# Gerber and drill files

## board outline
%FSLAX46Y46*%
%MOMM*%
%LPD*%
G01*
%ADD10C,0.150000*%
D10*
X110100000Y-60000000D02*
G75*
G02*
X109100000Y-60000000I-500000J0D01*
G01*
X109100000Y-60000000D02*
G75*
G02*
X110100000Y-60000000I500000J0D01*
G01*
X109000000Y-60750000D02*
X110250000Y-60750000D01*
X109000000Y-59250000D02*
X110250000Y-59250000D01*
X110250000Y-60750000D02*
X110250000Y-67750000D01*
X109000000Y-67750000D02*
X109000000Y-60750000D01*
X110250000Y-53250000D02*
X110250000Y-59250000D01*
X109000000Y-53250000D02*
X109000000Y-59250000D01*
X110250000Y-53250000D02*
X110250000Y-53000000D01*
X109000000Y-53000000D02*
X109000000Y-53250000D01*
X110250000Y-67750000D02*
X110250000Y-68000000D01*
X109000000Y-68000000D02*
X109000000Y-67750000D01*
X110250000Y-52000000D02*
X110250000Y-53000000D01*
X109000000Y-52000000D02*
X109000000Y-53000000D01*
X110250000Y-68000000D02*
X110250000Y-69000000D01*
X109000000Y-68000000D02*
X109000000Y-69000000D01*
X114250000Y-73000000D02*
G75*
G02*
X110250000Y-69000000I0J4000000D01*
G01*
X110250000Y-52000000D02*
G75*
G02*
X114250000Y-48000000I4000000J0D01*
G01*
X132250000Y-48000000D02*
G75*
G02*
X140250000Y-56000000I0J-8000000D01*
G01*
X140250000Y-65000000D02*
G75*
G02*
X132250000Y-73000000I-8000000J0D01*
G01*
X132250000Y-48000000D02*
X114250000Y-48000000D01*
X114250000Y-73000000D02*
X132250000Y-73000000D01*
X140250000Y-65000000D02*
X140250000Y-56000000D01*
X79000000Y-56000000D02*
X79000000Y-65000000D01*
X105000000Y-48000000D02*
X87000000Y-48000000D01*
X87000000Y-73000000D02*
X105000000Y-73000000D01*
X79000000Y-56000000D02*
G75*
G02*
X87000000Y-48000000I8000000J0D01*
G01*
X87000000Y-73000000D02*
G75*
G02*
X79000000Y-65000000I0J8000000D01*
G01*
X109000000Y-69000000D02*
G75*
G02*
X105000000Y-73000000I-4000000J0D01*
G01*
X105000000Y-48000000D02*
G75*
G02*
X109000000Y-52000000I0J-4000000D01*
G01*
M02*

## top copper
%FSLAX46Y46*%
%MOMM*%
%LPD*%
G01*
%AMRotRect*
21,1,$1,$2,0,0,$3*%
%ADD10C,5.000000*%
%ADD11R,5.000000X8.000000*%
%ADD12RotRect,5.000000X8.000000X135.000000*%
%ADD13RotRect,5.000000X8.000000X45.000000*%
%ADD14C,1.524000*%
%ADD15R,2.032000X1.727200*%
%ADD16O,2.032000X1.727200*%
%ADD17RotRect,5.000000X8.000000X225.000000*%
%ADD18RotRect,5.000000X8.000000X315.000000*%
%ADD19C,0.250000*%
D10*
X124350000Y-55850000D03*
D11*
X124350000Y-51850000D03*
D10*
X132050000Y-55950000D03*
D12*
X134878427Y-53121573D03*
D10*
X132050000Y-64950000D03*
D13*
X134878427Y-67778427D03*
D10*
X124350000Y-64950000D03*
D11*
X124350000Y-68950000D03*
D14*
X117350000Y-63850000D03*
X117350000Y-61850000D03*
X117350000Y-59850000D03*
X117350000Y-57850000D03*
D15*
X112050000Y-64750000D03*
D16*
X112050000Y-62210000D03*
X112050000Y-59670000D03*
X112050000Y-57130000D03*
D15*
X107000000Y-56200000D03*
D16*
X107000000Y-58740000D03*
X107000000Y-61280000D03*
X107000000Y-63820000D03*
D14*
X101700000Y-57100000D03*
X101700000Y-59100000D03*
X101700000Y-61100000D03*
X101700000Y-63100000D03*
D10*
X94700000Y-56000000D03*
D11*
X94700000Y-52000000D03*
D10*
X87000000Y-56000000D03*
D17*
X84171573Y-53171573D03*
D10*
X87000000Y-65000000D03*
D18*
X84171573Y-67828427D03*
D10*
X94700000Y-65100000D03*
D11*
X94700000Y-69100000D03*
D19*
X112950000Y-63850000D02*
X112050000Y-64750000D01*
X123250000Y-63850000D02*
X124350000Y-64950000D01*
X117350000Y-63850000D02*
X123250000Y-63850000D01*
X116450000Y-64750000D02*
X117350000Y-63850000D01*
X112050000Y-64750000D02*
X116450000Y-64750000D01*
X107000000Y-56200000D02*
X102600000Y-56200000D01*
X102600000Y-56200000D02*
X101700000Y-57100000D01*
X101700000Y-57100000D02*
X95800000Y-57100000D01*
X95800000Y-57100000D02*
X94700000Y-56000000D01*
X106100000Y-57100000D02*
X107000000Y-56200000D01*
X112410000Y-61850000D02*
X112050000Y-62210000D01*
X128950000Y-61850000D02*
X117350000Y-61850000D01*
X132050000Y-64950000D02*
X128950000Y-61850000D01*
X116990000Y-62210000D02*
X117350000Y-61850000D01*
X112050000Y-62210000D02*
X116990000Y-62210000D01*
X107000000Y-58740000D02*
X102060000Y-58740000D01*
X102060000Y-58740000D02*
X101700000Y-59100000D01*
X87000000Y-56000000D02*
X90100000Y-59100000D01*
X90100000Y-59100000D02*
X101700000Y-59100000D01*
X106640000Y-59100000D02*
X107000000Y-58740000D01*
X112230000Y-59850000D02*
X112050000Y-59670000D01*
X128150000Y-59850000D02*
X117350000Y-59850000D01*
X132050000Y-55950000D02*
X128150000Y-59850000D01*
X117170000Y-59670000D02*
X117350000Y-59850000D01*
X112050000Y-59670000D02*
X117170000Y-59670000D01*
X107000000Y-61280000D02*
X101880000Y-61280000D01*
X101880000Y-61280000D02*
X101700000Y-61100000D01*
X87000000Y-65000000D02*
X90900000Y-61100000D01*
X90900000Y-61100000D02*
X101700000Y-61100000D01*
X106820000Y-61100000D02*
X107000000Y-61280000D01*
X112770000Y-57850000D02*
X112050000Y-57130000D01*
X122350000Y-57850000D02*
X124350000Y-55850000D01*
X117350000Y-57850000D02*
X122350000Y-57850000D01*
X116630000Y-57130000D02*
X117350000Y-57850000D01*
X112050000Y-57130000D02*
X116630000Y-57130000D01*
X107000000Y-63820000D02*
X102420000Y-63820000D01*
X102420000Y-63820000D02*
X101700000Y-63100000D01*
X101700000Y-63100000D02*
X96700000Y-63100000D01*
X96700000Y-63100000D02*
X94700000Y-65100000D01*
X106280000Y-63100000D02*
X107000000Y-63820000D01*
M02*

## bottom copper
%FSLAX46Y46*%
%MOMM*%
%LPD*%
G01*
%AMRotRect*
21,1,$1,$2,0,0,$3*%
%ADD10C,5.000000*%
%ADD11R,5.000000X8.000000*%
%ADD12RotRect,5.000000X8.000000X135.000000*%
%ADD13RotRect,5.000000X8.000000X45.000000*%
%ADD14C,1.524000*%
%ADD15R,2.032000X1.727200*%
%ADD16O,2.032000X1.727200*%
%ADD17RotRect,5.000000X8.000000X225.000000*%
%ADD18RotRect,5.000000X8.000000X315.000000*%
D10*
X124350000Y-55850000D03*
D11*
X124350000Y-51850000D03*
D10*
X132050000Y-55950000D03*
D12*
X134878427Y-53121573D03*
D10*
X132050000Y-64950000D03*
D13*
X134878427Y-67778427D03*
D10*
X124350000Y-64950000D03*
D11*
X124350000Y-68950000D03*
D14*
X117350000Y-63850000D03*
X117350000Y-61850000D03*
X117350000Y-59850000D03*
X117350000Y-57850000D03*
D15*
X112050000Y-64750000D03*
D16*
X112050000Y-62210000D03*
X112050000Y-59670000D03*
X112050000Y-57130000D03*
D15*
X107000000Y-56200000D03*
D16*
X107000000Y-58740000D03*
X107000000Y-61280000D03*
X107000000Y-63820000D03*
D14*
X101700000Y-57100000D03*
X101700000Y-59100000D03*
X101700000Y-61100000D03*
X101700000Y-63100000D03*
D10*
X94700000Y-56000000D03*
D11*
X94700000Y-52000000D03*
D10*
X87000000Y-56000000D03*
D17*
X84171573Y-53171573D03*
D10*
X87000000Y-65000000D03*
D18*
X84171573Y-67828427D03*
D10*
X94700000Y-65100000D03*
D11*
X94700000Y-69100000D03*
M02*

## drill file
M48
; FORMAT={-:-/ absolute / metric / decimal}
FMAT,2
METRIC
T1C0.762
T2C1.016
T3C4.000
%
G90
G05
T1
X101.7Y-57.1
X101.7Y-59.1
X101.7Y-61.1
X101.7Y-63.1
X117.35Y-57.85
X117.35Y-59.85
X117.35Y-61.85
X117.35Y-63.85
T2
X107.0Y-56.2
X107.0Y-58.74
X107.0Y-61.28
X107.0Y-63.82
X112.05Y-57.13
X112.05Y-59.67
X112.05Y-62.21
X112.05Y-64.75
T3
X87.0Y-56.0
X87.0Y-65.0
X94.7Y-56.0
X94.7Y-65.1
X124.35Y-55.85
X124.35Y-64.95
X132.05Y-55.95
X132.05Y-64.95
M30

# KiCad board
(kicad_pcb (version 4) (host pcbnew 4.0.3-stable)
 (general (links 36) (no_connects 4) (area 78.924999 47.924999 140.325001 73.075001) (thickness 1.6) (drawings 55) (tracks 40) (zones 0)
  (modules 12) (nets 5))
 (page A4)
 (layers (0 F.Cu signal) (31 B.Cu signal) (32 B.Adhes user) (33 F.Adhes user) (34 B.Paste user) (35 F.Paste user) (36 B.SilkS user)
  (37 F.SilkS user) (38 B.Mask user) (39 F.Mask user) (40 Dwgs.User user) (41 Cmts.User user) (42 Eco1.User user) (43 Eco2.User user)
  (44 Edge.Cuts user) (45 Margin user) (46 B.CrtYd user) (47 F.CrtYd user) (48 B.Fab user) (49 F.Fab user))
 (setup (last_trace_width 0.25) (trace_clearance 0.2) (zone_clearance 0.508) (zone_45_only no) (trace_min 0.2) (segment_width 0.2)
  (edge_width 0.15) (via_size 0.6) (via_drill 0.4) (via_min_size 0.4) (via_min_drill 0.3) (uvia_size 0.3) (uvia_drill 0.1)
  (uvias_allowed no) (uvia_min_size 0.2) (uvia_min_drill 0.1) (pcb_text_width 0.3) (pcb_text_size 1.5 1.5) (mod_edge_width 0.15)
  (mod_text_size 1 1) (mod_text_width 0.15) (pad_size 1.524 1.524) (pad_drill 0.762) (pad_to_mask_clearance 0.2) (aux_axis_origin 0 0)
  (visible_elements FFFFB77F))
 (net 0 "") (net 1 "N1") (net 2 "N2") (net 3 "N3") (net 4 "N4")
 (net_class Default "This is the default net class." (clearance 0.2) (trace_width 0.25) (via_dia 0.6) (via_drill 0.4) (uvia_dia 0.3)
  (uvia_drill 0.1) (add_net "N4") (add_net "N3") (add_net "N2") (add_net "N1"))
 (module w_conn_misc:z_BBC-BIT (layer F.Cu) (at 124.35 55.85 180)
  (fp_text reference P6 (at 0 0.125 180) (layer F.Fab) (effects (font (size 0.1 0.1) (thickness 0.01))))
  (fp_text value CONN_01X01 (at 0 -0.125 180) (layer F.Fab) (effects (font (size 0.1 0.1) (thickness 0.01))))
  (pad 1 thru_hole circle (at 0 0 180) (size 5 5) (drill 4) (layers *.Cu *.Mask) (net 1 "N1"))
  (pad 1 smd rect (at 0 4 180) (size 5 8) (layers F.Cu F.Mask) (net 1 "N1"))
  (pad 1 smd rect (at 0 4 180) (size 5 8) (layers *.Mask B.Cu) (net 1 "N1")))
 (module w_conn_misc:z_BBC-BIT (layer F.Cu) (at 132.05 55.95 135)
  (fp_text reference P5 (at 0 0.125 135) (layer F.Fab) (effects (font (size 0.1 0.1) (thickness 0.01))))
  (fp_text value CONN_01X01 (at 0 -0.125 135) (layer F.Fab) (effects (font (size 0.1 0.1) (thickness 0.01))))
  (pad 1 thru_hole circle (at 0 0 135) (size 5 5) (drill 4) (layers *.Cu *.Mask) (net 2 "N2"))
  (pad 1 smd rect (at 0 4 135) (size 5 8) (layers F.Cu F.Mask) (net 2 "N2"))
  (pad 1 smd rect (at 0 4 135) (size 5 8) (layers *.Mask B.Cu) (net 2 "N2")))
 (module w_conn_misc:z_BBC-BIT (layer F.Cu) (at 132.05 64.95 45)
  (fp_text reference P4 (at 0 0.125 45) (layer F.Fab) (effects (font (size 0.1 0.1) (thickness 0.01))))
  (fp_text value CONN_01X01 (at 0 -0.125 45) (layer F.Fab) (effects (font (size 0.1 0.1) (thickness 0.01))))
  (pad 1 thru_hole circle (at 0 0 45) (size 5 5) (drill 4) (layers *.Cu *.Mask) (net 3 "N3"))
  (pad 1 smd rect (at 0 4 45) (size 5 8) (layers F.Cu F.Mask) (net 3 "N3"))
  (pad 1 smd rect (at 0 4 45) (size 5 8) (layers *.Mask B.Cu) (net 3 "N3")))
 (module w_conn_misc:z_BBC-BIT (layer F.Cu) (at 124.35 64.95)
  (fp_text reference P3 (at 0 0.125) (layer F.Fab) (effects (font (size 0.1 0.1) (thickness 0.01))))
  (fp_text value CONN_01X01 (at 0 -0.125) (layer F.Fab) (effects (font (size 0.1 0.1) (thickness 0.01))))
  (pad 1 thru_hole circle (at 0 0) (size 5 5) (drill 4) (layers *.Cu *.Mask) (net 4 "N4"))
  (pad 1 smd rect (at 0 4) (size 5 8) (layers F.Cu F.Mask) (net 4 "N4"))
  (pad 1 smd rect (at 0 4) (size 5 8) (layers *.Mask B.Cu) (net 4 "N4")))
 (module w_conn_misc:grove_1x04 (layer F.Cu) (at 117.35 63.85 180)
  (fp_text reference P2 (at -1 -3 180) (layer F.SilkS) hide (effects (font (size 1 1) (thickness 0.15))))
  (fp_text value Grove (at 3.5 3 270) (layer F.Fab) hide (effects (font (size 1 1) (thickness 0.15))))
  (pad 1 thru_hole circle (at 0 0 180) (size 1.524 1.524) (drill 0.762) (layers *.Cu *.Mask F.SilkS) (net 4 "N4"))
  (pad 2 thru_hole circle (at 0 2 180) (size 1.524 1.524) (drill 0.762) (layers *.Cu *.Mask F.SilkS) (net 3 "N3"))
  (pad 3 thru_hole circle (at 0 4 180) (size 1.524 1.524) (drill 0.762) (layers *.Cu *.Mask F.SilkS) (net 2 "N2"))
  (pad 4 thru_hole circle (at 0 6 180) (size 1.524 1.524) (drill 0.762) (layers *.Cu *.Mask F.SilkS) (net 1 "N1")))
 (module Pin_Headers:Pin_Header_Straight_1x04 (layer F.Cu) (at 112.05 64.75 180)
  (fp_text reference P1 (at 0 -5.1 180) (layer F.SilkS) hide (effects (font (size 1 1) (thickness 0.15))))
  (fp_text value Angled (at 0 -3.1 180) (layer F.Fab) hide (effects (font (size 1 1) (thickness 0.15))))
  (pad 1 thru_hole rect (at 0 0 180) (size 2.032 1.7272) (drill 1.016) (layers *.Cu *.Mask F.SilkS) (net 4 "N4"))
  (pad 2 thru_hole oval (at 0 2.54 180) (size 2.032 1.7272) (drill 1.016) (layers *.Cu *.Mask F.SilkS) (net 3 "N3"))
  (pad 3 thru_hole oval (at 0 5.08 180) (size 2.032 1.7272) (drill 1.016) (layers *.Cu *.Mask F.SilkS) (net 2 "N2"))
  (pad 4 thru_hole oval (at 0 7.62 180) (size 2.032 1.7272) (drill 1.016) (layers *.Cu *.Mask F.SilkS) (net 1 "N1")))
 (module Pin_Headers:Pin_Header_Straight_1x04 (layer F.Cu) (at 107 56.2)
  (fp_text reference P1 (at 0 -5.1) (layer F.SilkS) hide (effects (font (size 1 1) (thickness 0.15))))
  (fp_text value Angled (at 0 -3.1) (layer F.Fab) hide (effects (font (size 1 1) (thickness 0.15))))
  (pad 1 thru_hole rect (at 0 0) (size 2.032 1.7272) (drill 1.016) (layers *.Cu *.Mask F.SilkS) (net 4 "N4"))
  (pad 2 thru_hole oval (at 0 2.54) (size 2.032 1.7272) (drill 1.016) (layers *.Cu *.Mask F.SilkS) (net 3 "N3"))
  (pad 3 thru_hole oval (at 0 5.08) (size 2.032 1.7272) (drill 1.016) (layers *.Cu *.Mask F.SilkS) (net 2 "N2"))
  (pad 4 thru_hole oval (at 0 7.62) (size 2.032 1.7272) (drill 1.016) (layers *.Cu *.Mask F.SilkS) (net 1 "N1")))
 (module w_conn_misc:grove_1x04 (layer F.Cu) (at 101.7 57.1)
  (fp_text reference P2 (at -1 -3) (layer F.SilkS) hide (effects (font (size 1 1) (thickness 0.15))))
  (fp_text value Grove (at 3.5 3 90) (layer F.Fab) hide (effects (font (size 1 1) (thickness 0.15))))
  (pad 1 thru_hole circle (at 0 0) (size 1.524 1.524) (drill 0.762) (layers *.Cu *.Mask F.SilkS) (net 4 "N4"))
  (pad 2 thru_hole circle (at 0 2) (size 1.524 1.524) (drill 0.762) (layers *.Cu *.Mask F.SilkS) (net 3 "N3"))
  (pad 3 thru_hole circle (at 0 4) (size 1.524 1.524) (drill 0.762) (layers *.Cu *.Mask F.SilkS) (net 2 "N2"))
  (pad 4 thru_hole circle (at 0 6) (size 1.524 1.524) (drill 0.762) (layers *.Cu *.Mask F.SilkS) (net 1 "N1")))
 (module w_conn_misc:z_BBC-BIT (layer F.Cu) (at 94.7 56 180)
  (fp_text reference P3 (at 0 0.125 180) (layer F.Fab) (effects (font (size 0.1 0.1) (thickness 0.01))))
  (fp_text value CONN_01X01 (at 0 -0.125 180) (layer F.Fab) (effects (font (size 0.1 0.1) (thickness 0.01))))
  (pad 1 thru_hole circle (at 0 0 180) (size 5 5) (drill 4) (layers *.Cu *.Mask) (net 4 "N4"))
  (pad 1 smd rect (at 0 4 180) (size 5 8) (layers F.Cu F.Mask) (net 4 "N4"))
  (pad 1 smd rect (at 0 4 180) (size 5 8) (layers *.Mask B.Cu) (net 4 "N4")))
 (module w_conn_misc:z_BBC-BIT (layer F.Cu) (at 87 56 225)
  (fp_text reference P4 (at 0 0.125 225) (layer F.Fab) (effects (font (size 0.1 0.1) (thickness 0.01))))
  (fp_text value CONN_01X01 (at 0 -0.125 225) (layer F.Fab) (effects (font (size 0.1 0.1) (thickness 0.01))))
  (pad 1 thru_hole circle (at 0 0 225) (size 5 5) (drill 4) (layers *.Cu *.Mask) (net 3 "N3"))
  (pad 1 smd rect (at 0 4 225) (size 5 8) (layers F.Cu F.Mask) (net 3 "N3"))
  (pad 1 smd rect (at 0 4 225) (size 5 8) (layers *.Mask B.Cu) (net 3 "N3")))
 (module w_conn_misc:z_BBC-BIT (layer F.Cu) (at 87 65 315)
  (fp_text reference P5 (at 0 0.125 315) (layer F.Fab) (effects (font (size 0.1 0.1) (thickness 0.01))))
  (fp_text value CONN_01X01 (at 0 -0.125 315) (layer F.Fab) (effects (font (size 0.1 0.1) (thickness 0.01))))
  (pad 1 thru_hole circle (at 0 0 315) (size 5 5) (drill 4) (layers *.Cu *.Mask) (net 2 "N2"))
  (pad 1 smd rect (at 0 4 315) (size 5 8) (layers F.Cu F.Mask) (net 2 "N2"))
  (pad 1 smd rect (at 0 4 315) (size 5 8) (layers *.Mask B.Cu) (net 2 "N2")))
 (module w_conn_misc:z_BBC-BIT (layer F.Cu) (at 94.7 65.1)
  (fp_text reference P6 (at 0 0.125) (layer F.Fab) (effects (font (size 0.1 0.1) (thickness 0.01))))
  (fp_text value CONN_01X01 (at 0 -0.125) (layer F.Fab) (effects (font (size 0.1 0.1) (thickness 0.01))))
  (pad 1 thru_hole circle (at 0 0) (size 5 5) (drill 4) (layers *.Cu *.Mask) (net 1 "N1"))
  (pad 1 smd rect (at 0 4) (size 5 8) (layers F.Cu F.Mask) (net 1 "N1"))
  (pad 1 smd rect (at 0 4) (size 5 8) (layers *.Mask B.Cu) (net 1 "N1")))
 (gr_circle (center 109.6 60) (end 110.1 60) (layer Edge.Cuts) (width 0.15))
 (gr_line (start 109 60.75) (end 110.25 60.75) (angle 90) (layer Edge.Cuts) (width 0.15))
 (gr_line (start 109 59.25) (end 110.25 59.25) (angle 90) (layer Edge.Cuts) (width 0.15))
 (gr_line (start 110.25 60.75) (end 110.25 67.75) (angle 90) (layer Edge.Cuts) (width 0.15))
 (gr_line (start 109 67.75) (end 109 60.75) (angle 90) (layer Edge.Cuts) (width 0.15))
 (gr_line (start 110.25 53.25) (end 110.25 59.25) (angle 90) (layer Edge.Cuts) (width 0.15))
 (gr_line (start 109 53.25) (end 109 59.25) (angle 90) (layer Edge.Cuts) (width 0.15))
 (gr_line (start 110.25 53.25) (end 110.25 53) (angle 90) (layer Edge.Cuts) (width 0.15))
 (gr_line (start 109 53) (end 109 53.25) (angle 90) (layer Edge.Cuts) (width 0.15))
 (gr_line (start 110.25 67.75) (end 110.25 68) (angle 90) (layer Edge.Cuts) (width 0.15))
 (gr_line (start 109 68) (end 109 67.75) (angle 90) (layer Edge.Cuts) (width 0.15))
 (gr_line (start 110.25 52) (end 110.25 53) (angle 90) (layer Edge.Cuts) (width 0.15))
 (gr_line (start 109 52) (end 109 53) (angle 90) (layer Edge.Cuts) (width 0.15))
 (gr_line (start 110.25 68) (end 110.25 69) (angle 90) (layer Edge.Cuts) (width 0.15))
 (gr_line (start 109 68) (end 109 69) (angle 90) (layer Edge.Cuts) (width 0.15))
 (gr_arc (start 114.25 69) (end 114.25 73) (angle 90) (layer Edge.Cuts) (width 0.15))
 (gr_arc (start 114.25 52) (end 110.25 52) (angle 90) (layer Edge.Cuts) (width 0.15))
 (gr_arc (start 132.25 56) (end 132.25 48) (angle 90) (layer Edge.Cuts) (width 0.15))
 (gr_arc (start 132.25 65) (end 140.25 65) (angle 90) (layer Edge.Cuts) (width 0.15))
 (gr_line (start 132.25 48) (end 114.25 48) (angle 90) (layer Edge.Cuts) (width 0.15))
 (gr_line (start 114.25 73) (end 132.25 73) (angle 90) (layer Edge.Cuts) (width 0.15))
 (gr_line (start 140.25 65) (end 140.25 56) (angle 90) (layer Edge.Cuts) (width 0.15))
 (gr_line (start 79 56) (end 79 65) (angle 90) (layer Edge.Cuts) (width 0.15))
 (gr_line (start 105 48) (end 87 48) (angle 90) (layer Edge.Cuts) (width 0.15))
 (gr_line (start 87 73) (end 105 73) (angle 90) (layer Edge.Cuts) (width 0.15))
 (gr_arc (start 87 56) (end 79 56) (angle 90) (layer Edge.Cuts) (width 0.15))
 (gr_arc (start 87 65) (end 87 73) (angle 90) (layer Edge.Cuts) (width 0.15))
 (gr_arc (start 105 69) (end 109 69) (angle 90) (layer Edge.Cuts) (width 0.15))
 (gr_arc (start 105 52) (end 105 48) (angle 90) (layer Edge.Cuts) (width 0.15))
 (segment (start 112.95 63.85) (end 112.05 64.75) (width 0.25) (layer F.Cu) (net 4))
 (segment (start 123.25 63.85) (end 124.35 64.95) (width 0.25) (layer F.Cu) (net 4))
 (segment (start 117.35 63.85) (end 123.25 63.85) (width 0.25) (layer F.Cu) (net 4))
 (segment (start 116.45 64.75) (end 117.35 63.85) (width 0.25) (layer F.Cu) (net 4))
 (segment (start 112.05 64.75) (end 116.45 64.75) (width 0.25) (layer F.Cu) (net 4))
 (segment (start 107 56.2) (end 102.6 56.2) (width 0.25) (layer F.Cu) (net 4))
 (segment (start 102.6 56.2) (end 101.7 57.1) (width 0.25) (layer F.Cu) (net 4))
 (segment (start 101.7 57.1) (end 95.8 57.1) (width 0.25) (layer F.Cu) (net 4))
 (segment (start 95.8 57.1) (end 94.7 56) (width 0.25) (layer F.Cu) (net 4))
 (segment (start 106.1 57.1) (end 107 56.2) (width 0.25) (layer F.Cu) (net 4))
 (segment (start 112.41 61.85) (end 112.05 62.21) (width 0.25) (layer F.Cu) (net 3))
 (segment (start 128.95 61.85) (end 117.35 61.85) (width 0.25) (layer F.Cu) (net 3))
 (segment (start 132.05 64.95) (end 128.95 61.85) (width 0.25) (layer F.Cu) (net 3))
 (segment (start 116.99 62.21) (end 117.35 61.85) (width 0.25) (layer F.Cu) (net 3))
 (segment (start 112.05 62.21) (end 116.99 62.21) (width 0.25) (layer F.Cu) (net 3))
 (segment (start 107 58.74) (end 102.06 58.74) (width 0.25) (layer F.Cu) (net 3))
 (segment (start 102.06 58.74) (end 101.7 59.1) (width 0.25) (layer F.Cu) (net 3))
 (segment (start 87 56) (end 90.1 59.1) (width 0.25) (layer F.Cu) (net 3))
 (segment (start 90.1 59.1) (end 101.7 59.1) (width 0.25) (layer F.Cu) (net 3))
 (segment (start 106.64 59.1) (end 107 58.74) (width 0.25) (layer F.Cu) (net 3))
 (segment (start 112.23 59.85) (end 112.05 59.67) (width 0.25) (layer F.Cu) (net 2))
 (segment (start 128.15 59.85) (end 117.35 59.85) (width 0.25) (layer F.Cu) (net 2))
 (segment (start 132.05 55.95) (end 128.15 59.85) (width 0.25) (layer F.Cu) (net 2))
 (segment (start 117.17 59.67) (end 117.35 59.85) (width 0.25) (layer F.Cu) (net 2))
 (segment (start 112.05 59.67) (end 117.17 59.67) (width 0.25) (layer F.Cu) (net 2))
 (segment (start 107 61.28) (end 101.88 61.28) (width 0.25) (layer F.Cu) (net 2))
 (segment (start 101.88 61.28) (end 101.7 61.1) (width 0.25) (layer F.Cu) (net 2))
 (segment (start 87 65) (end 90.9 61.1) (width 0.25) (layer F.Cu) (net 2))
 (segment (start 90.9 61.1) (end 101.7 61.1) (width 0.25) (layer F.Cu) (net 2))
 (segment (start 106.82 61.1) (end 107 61.28) (width 0.25) (layer F.Cu) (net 2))
 (segment (start 112.77 57.85) (end 112.05 57.13) (width 0.25) (layer F.Cu) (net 1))
 (segment (start 122.35 57.85) (end 124.35 55.85) (width 0.25) (layer F.Cu) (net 1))
 (segment (start 117.35 57.85) (end 122.35 57.85) (width 0.25) (layer F.Cu) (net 1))
 (segment (start 116.63 57.13) (end 117.35 57.85) (width 0.25) (layer F.Cu) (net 1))
 (segment (start 112.05 57.13) (end 116.63 57.13) (width 0.25) (layer F.Cu) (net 1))
 (segment (start 107 63.82) (end 102.42 63.82) (width 0.25) (layer F.Cu) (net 1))
 (segment (start 102.42 63.82) (end 101.7 63.1) (width 0.25) (layer F.Cu) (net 1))
 (segment (start 101.7 63.1) (end 96.7 63.1) (width 0.25) (layer F.Cu) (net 1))
 (segment (start 96.7 63.1) (end 94.7 65.1) (width 0.25) (layer F.Cu) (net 1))
 (segment (start 106.28 63.1) (end 107 63.82) (width 0.25) (layer F.Cu) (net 1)))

